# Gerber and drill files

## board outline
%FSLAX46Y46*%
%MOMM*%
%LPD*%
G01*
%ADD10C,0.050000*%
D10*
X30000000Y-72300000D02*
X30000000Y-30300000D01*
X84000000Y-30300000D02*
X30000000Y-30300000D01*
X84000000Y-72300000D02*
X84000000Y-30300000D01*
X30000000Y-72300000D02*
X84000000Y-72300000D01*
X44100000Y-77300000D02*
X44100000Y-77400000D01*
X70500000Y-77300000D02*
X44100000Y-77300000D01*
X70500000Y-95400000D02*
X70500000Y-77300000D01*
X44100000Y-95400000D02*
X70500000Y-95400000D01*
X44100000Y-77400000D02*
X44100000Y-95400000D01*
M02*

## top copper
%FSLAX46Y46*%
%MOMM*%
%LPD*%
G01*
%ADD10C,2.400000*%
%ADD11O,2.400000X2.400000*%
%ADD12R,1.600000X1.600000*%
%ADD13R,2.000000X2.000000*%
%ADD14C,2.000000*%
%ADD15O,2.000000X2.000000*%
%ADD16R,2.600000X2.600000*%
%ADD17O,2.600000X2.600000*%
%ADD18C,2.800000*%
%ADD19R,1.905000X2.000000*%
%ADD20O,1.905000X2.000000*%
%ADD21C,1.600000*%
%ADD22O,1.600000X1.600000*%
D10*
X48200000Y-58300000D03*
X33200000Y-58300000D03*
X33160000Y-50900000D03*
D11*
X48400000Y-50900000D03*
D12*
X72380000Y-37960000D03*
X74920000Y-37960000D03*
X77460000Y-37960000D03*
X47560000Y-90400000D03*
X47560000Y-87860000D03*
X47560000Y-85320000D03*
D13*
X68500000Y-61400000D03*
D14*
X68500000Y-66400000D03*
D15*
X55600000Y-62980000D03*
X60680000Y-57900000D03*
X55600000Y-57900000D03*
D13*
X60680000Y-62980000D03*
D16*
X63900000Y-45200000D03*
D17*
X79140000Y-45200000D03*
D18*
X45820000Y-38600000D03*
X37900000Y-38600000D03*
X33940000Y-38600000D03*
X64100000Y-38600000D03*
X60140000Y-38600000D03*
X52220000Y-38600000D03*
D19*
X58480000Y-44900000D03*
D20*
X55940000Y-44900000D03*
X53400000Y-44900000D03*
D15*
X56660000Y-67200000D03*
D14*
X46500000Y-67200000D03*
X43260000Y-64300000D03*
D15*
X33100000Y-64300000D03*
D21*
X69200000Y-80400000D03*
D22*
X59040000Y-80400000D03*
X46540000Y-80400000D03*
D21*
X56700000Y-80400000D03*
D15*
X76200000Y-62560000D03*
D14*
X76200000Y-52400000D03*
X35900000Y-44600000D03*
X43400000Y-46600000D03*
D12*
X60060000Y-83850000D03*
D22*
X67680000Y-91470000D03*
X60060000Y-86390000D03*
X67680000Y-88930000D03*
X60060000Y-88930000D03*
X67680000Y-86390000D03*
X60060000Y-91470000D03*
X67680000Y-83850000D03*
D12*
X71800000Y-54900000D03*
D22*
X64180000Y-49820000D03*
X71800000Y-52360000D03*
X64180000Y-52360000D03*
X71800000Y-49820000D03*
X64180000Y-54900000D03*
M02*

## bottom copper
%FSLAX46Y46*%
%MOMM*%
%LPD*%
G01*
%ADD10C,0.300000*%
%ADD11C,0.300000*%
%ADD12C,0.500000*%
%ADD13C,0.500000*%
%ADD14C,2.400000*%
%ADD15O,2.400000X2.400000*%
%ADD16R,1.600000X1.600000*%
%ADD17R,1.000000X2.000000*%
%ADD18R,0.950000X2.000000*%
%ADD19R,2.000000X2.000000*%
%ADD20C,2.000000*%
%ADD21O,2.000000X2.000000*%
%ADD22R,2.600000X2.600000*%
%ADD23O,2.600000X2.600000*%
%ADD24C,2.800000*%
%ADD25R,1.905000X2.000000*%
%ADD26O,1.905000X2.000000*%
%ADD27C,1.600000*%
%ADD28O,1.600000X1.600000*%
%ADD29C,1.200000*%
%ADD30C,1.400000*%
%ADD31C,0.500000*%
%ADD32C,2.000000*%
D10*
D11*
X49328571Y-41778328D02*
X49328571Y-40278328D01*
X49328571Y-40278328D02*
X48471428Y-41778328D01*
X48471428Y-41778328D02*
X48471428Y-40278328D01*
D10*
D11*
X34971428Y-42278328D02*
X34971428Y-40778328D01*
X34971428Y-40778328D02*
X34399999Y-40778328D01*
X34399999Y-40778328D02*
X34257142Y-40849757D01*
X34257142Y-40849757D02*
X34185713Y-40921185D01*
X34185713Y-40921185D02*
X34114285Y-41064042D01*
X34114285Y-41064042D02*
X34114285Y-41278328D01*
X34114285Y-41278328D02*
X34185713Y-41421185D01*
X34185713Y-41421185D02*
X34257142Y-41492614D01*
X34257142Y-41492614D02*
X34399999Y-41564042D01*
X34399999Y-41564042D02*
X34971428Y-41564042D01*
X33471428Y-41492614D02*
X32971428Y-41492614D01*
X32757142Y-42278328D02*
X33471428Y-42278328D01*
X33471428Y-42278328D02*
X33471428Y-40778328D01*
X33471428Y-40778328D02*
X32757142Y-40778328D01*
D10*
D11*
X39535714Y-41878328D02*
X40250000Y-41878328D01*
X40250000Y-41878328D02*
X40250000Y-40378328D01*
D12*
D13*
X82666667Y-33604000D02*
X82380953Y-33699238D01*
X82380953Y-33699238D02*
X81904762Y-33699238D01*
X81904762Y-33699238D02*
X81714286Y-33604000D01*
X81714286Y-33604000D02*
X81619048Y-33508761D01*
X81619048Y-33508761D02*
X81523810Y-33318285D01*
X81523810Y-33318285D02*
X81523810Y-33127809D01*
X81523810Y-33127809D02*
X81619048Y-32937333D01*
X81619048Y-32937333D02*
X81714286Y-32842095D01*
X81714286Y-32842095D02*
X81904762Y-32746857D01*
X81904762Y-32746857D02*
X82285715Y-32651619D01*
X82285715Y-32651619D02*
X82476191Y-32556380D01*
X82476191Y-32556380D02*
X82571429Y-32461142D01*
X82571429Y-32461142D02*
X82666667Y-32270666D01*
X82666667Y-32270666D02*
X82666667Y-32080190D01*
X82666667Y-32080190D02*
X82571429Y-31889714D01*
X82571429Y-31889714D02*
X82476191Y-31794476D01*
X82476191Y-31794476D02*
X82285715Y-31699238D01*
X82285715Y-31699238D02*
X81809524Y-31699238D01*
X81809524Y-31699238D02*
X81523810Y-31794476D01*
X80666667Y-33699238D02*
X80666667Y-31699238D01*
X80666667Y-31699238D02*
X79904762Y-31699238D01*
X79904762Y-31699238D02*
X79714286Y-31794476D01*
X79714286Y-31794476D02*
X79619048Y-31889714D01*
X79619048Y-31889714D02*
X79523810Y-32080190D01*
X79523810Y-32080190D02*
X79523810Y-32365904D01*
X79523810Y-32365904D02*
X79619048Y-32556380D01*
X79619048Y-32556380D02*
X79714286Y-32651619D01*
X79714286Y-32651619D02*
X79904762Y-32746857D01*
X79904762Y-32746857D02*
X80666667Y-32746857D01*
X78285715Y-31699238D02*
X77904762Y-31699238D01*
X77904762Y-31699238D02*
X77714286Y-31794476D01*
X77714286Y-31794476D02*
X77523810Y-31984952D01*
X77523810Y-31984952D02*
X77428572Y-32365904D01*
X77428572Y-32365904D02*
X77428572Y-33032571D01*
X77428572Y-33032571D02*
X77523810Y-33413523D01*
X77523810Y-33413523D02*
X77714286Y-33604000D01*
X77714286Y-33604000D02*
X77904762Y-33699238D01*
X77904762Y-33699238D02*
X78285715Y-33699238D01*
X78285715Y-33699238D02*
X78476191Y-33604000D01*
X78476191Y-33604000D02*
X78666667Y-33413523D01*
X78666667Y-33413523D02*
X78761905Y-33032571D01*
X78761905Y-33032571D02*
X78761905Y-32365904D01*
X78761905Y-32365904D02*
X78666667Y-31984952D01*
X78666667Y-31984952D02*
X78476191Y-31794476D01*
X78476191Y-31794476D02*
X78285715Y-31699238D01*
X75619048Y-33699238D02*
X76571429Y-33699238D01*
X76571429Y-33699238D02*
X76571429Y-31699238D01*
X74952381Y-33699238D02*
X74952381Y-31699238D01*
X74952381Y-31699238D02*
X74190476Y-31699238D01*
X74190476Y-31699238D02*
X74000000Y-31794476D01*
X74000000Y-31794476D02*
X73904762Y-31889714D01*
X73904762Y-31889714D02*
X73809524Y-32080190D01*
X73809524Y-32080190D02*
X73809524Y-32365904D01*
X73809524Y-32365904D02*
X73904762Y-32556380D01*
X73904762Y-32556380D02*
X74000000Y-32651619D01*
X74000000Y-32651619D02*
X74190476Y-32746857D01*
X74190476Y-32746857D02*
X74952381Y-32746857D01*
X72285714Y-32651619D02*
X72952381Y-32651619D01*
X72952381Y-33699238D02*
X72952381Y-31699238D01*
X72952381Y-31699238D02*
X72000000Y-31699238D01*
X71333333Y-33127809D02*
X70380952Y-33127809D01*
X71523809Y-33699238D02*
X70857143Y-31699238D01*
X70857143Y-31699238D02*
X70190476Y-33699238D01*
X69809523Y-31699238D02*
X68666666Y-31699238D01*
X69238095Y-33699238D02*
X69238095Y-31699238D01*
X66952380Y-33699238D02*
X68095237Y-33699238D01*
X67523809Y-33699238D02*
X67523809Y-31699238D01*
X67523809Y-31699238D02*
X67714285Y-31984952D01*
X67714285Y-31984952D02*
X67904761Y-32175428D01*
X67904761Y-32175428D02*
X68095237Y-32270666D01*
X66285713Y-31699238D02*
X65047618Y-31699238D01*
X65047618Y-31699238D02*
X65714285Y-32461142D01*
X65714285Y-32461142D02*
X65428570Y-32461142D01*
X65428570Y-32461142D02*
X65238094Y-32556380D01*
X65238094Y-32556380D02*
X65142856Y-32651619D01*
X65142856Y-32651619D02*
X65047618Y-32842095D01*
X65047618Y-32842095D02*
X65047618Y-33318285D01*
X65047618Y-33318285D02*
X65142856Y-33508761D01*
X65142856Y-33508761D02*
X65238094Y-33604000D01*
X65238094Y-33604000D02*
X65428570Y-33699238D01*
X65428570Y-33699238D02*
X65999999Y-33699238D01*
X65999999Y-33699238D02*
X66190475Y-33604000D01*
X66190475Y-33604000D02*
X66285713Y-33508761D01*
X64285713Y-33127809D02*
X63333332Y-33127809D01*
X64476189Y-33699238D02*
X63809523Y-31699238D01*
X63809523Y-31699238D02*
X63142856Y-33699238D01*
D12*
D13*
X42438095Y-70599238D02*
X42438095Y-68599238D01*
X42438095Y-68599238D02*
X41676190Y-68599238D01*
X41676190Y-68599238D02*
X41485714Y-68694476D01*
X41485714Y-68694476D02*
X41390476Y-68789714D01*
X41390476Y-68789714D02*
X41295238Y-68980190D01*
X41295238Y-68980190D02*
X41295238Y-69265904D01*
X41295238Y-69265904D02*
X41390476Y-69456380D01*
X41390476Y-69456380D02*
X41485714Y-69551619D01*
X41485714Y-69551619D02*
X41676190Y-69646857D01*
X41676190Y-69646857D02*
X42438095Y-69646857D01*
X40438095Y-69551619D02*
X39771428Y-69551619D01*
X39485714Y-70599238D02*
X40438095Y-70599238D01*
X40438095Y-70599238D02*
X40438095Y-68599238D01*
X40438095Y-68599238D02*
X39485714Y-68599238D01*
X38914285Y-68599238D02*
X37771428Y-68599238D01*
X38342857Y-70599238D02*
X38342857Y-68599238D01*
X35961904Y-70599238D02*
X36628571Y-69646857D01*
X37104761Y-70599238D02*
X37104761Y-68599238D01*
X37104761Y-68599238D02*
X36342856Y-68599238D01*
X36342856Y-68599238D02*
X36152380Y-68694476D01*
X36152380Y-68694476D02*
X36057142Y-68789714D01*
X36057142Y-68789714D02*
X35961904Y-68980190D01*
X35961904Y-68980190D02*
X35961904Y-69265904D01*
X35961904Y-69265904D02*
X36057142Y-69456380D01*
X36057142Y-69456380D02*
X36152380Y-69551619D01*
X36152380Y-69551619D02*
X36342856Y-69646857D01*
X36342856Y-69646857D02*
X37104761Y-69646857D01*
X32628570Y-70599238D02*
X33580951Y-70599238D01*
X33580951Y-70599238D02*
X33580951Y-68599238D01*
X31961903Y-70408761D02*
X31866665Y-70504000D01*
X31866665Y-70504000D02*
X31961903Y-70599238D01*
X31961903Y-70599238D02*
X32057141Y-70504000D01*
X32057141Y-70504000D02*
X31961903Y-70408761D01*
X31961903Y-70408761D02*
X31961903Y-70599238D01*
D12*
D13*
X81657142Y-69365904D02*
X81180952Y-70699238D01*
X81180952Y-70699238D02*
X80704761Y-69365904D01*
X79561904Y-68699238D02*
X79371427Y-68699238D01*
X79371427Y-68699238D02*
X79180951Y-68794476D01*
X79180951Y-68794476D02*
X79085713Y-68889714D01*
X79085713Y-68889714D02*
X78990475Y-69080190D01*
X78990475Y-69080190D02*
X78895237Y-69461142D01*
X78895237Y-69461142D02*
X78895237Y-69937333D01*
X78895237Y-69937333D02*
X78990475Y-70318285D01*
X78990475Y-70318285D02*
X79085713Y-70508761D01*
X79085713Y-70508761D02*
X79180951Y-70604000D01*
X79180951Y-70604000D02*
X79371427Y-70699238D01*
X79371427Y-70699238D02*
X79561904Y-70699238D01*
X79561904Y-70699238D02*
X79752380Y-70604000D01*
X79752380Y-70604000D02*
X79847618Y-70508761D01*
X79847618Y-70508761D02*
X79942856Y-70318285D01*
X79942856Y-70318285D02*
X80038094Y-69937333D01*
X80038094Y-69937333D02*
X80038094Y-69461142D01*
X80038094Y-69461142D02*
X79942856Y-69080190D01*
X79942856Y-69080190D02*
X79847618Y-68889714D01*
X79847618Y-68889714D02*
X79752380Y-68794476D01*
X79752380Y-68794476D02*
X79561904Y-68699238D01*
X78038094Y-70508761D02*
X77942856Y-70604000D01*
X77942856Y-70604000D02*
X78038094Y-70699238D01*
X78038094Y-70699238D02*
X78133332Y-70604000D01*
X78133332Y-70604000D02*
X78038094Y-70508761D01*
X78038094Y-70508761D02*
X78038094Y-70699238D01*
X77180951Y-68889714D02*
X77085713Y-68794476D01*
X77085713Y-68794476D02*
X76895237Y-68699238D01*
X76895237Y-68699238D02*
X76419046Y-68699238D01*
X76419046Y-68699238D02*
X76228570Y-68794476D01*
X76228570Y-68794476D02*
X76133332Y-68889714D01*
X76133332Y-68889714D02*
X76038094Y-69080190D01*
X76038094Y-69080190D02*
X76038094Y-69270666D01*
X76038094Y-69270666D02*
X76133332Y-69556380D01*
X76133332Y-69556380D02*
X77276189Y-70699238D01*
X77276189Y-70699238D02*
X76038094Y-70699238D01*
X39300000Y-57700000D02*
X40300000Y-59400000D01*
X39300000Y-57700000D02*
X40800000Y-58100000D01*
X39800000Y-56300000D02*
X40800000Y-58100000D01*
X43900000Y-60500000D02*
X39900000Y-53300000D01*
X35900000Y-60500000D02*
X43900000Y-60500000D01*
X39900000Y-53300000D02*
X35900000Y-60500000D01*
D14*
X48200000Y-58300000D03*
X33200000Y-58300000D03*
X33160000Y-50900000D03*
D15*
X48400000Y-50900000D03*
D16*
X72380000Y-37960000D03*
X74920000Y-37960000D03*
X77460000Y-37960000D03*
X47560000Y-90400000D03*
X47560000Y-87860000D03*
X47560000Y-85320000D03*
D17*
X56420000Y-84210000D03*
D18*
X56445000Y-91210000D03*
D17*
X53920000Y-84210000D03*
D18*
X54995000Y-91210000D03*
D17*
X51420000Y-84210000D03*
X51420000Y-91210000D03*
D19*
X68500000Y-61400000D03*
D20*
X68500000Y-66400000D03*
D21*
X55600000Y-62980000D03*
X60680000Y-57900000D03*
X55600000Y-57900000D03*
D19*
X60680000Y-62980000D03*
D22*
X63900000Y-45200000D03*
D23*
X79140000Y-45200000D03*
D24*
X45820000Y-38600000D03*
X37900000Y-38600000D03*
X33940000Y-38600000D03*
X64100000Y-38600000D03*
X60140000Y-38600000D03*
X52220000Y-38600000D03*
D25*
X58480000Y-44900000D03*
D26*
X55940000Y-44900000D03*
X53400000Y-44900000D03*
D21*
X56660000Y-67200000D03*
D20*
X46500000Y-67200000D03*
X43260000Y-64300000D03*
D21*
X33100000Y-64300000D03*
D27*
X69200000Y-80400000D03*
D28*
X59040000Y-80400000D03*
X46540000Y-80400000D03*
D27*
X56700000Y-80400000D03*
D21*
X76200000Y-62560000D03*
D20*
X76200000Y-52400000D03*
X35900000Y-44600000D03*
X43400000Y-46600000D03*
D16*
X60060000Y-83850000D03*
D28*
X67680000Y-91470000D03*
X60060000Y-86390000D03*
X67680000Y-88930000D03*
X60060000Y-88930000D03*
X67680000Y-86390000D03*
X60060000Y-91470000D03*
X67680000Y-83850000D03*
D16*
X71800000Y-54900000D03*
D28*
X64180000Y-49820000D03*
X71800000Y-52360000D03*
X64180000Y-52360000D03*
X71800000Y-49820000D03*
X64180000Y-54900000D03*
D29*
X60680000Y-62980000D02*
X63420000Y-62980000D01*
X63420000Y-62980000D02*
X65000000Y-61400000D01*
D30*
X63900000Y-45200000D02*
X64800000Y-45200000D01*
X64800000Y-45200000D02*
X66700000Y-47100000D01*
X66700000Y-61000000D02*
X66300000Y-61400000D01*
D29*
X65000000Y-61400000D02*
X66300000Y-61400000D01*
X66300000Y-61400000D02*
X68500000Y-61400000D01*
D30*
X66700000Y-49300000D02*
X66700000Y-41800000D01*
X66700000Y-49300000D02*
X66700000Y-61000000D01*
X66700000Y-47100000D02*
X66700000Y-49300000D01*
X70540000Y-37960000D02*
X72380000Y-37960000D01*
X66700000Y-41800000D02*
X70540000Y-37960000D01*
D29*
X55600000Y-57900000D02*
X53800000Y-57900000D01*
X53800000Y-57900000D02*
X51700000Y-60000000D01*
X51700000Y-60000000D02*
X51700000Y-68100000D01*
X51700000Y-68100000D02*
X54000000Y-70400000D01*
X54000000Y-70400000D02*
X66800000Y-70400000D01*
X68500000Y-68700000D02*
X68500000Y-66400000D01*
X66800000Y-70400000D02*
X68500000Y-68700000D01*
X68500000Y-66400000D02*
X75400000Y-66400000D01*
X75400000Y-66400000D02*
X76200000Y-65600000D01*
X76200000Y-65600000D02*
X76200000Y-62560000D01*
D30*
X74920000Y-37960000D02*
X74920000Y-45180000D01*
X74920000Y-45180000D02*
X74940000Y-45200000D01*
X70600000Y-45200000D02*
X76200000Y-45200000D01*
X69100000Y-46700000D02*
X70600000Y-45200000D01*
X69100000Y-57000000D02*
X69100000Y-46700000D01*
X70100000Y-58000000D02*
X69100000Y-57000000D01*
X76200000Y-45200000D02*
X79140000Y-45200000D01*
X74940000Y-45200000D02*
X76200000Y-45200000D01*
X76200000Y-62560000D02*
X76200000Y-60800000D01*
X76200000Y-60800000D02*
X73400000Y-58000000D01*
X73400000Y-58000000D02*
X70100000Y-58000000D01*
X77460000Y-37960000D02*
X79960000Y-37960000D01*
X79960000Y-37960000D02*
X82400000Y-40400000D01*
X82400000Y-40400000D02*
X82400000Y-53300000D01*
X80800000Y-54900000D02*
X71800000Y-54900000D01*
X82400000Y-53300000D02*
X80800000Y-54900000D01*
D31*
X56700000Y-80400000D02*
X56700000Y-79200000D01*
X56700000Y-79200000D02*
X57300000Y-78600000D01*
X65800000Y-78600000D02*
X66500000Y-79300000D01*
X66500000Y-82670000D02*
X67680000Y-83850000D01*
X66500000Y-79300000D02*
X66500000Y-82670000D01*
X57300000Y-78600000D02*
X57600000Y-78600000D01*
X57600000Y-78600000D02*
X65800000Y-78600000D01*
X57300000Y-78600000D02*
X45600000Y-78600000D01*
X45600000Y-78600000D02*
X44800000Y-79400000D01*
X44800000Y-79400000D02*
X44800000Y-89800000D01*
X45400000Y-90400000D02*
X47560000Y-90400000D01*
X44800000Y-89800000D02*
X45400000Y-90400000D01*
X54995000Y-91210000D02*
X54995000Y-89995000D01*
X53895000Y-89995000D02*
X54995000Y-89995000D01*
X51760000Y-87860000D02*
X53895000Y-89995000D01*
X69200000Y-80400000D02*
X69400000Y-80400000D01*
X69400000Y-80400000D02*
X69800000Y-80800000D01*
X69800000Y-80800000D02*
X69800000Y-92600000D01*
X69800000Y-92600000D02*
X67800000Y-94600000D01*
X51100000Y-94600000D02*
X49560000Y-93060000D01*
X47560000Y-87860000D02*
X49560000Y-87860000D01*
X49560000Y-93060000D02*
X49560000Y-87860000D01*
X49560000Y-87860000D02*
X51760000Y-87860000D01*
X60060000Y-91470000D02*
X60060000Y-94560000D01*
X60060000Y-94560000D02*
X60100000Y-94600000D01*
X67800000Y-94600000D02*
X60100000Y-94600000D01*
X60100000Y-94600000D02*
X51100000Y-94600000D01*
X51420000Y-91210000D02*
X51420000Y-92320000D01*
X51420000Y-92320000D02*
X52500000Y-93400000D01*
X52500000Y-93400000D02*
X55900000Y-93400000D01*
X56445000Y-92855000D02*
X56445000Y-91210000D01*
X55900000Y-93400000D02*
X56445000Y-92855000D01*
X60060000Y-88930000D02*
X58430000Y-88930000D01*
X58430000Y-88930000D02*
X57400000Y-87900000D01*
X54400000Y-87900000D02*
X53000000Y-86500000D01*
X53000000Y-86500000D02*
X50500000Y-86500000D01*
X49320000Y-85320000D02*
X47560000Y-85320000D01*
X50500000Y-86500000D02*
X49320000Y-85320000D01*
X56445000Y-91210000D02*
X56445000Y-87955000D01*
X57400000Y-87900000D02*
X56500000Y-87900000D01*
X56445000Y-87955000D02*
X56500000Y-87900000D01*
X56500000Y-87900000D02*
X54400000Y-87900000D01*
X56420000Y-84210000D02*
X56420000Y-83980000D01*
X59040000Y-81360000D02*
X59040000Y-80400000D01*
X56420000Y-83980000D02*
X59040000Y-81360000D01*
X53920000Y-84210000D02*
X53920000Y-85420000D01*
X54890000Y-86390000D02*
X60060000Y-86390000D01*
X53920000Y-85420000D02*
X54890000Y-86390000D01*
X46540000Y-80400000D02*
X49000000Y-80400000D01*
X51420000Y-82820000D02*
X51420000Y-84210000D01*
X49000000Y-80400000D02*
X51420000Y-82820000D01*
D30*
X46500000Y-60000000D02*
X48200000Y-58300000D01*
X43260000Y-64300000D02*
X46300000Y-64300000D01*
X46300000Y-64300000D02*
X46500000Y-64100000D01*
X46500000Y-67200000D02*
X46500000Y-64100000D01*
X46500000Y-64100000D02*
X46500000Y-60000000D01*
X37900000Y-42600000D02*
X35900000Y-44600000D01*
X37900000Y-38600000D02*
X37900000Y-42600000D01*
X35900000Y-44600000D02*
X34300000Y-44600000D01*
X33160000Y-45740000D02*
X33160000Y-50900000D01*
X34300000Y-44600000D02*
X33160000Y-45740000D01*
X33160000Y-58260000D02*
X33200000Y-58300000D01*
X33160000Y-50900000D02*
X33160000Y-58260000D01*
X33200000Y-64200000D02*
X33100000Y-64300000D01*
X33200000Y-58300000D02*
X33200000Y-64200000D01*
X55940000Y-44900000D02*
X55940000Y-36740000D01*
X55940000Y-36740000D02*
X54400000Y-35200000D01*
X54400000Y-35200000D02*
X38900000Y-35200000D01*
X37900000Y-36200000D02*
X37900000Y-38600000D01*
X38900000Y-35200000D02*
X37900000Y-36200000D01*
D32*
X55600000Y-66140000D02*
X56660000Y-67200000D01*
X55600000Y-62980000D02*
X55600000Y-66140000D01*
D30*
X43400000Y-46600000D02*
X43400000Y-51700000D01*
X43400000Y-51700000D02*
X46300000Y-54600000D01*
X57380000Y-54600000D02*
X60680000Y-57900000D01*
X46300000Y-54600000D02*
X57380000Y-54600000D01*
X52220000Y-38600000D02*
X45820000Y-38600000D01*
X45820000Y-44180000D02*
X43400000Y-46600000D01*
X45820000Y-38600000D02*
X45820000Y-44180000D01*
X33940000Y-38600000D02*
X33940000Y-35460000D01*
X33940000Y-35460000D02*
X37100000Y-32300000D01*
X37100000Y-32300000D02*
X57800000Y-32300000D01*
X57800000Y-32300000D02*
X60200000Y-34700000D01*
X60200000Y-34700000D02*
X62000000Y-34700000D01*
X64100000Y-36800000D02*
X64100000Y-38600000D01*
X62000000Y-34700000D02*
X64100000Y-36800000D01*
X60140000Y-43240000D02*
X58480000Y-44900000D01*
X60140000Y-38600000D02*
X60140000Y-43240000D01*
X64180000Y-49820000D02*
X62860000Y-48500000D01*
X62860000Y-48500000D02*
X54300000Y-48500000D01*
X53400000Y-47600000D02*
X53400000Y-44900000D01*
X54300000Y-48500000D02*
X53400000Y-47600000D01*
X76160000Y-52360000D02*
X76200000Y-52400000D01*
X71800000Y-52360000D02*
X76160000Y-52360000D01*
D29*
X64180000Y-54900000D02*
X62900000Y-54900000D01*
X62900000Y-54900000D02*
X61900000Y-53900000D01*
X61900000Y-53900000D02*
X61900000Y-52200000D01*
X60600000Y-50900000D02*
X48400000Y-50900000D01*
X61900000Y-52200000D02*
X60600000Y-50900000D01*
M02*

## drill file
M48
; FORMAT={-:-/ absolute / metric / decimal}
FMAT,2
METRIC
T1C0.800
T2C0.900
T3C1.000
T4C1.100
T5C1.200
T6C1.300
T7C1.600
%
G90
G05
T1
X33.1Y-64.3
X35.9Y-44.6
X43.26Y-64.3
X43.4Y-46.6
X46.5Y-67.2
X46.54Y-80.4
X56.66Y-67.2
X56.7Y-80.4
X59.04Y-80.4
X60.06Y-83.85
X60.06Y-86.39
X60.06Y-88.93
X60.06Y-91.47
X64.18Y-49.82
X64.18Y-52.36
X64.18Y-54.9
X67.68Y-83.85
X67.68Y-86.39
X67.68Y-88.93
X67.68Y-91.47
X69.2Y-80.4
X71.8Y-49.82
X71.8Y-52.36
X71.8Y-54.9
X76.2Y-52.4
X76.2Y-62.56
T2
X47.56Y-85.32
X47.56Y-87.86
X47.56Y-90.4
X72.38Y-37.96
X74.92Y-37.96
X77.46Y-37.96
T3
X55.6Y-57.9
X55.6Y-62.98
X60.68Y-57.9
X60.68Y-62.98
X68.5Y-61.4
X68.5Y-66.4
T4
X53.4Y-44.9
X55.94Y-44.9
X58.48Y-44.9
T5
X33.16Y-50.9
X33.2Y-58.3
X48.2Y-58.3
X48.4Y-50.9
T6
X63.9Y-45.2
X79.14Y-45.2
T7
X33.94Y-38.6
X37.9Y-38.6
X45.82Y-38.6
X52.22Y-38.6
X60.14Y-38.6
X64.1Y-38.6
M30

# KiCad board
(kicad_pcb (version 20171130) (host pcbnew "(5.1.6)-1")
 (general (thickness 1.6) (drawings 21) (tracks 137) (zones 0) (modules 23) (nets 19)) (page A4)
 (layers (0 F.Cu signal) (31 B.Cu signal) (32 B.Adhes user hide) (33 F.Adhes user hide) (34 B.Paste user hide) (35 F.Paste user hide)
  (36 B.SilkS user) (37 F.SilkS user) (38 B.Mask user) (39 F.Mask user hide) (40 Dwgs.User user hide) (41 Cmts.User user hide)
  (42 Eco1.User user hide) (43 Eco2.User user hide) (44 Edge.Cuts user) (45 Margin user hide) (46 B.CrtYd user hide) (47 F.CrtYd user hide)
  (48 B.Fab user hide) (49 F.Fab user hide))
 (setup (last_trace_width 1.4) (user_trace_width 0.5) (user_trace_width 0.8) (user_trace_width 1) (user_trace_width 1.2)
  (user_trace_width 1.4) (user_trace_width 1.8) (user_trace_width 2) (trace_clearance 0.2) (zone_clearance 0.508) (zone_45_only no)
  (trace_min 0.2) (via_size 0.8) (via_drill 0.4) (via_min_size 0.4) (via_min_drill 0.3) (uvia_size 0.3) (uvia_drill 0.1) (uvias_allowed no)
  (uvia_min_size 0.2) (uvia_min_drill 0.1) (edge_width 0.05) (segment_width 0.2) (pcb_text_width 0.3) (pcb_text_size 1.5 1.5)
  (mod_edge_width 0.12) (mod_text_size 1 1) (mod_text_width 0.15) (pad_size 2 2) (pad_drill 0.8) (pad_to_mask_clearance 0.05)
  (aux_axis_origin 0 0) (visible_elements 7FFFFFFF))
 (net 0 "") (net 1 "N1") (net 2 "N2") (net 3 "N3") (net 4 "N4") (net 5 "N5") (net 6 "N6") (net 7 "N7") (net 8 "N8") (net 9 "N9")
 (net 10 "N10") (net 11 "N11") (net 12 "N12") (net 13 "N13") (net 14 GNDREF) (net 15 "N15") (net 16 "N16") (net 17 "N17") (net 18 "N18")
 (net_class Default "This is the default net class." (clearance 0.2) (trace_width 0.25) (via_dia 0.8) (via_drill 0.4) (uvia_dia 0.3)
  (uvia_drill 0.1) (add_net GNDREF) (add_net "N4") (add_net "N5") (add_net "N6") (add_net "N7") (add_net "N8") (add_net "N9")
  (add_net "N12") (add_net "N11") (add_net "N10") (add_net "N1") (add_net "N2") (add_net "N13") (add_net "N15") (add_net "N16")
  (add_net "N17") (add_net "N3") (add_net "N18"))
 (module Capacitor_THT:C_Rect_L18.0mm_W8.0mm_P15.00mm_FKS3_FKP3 (layer F.Cu) (at 48.2 58.3 180)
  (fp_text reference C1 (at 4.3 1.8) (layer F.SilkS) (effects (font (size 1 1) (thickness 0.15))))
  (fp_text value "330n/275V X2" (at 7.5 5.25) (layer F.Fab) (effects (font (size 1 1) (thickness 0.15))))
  (pad 1 thru_hole circle (at 0 0 180) (size 2.4 2.4) (drill 1.2) (layers *.Cu *.Mask) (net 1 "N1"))
  (pad 2 thru_hole circle (at 15 0 180) (size 2.4 2.4) (drill 1.2) (layers *.Cu *.Mask) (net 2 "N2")))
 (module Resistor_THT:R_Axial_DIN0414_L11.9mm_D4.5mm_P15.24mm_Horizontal (layer F.Cu) (at 33.16 50.9)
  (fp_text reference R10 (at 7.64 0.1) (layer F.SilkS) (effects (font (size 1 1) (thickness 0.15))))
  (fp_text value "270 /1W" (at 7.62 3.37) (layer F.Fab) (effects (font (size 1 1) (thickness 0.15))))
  (pad 1 thru_hole circle (at 0 0) (size 2.4 2.4) (drill 1.2) (layers *.Cu *.Mask) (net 2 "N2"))
  (pad 2 thru_hole oval (at 15.24 0) (size 2.4 2.4) (drill 1.2) (layers *.Cu *.Mask) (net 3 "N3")))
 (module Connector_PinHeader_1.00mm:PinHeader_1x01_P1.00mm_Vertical (layer F.Cu) (at 72.38 37.96)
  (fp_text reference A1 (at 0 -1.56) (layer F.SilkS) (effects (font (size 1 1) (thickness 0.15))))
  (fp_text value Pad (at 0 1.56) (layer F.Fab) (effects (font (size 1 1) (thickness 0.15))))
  (pad 1 thru_hole rect (at 0 0) (size 1.6 1.6) (drill 0.9) (layers *.Cu *.Mask) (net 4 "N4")))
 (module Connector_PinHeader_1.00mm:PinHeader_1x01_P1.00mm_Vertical (layer F.Cu) (at 74.92 37.96)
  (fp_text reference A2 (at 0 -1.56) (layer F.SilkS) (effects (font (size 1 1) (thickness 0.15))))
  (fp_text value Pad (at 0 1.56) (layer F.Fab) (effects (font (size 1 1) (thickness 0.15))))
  (pad 1 thru_hole rect (at 0 0) (size 1.6 1.6) (drill 0.9) (layers *.Cu *.Mask) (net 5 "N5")))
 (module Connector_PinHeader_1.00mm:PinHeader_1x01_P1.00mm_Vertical (layer F.Cu) (at 77.46 37.96)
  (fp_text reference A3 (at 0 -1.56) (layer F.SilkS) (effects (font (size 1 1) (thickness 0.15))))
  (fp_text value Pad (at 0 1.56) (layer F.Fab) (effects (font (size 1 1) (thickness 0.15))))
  (pad 1 thru_hole rect (at 0 0) (size 1.6 1.6) (drill 0.9) (layers *.Cu *.Mask) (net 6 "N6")))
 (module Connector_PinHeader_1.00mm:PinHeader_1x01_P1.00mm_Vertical (layer F.Cu) (at 47.56 90.4 90)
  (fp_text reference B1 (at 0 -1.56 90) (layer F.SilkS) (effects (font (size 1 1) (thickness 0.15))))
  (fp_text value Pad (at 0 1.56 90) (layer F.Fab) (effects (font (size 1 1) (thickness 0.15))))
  (pad 1 thru_hole rect (at 0 0 90) (size 1.6 1.6) (drill 0.9) (layers *.Cu *.Mask) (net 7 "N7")))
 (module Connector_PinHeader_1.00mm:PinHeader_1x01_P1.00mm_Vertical (layer F.Cu) (at 47.56 87.86 90)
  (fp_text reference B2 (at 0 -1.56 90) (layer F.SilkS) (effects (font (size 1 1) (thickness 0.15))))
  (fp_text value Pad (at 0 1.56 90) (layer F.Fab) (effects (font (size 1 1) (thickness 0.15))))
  (pad 1 thru_hole rect (at 0 0 90) (size 1.6 1.6) (drill 0.9) (layers *.Cu *.Mask) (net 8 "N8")))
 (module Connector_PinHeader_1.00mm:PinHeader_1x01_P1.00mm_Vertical (layer F.Cu) (at 47.56 85.32 90)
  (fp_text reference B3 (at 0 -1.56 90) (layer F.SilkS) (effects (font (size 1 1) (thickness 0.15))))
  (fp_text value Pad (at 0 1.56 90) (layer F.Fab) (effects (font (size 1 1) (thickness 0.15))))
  (pad 1 thru_hole rect (at 0 0 90) (size 1.6 1.6) (drill 0.9) (layers *.Cu *.Mask) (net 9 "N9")))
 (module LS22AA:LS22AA (layer B.Cu) (at 53.92 87.71)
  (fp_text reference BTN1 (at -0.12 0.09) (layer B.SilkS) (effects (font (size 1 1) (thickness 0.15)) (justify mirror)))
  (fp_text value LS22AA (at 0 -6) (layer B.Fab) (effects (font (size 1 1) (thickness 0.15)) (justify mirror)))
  (pad 6 smd rect (at 2.5 -3.5) (size 1 2) (layers B.Cu B.Paste B.Mask) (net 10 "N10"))
  (pad 5 smd rect (at 2.525 3.5) (size 0.95 2) (layers B.Cu B.Paste B.Mask) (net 9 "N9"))
  (pad 4 smd rect (at 0 -3.5) (size 1 2) (layers B.Cu B.Paste B.Mask) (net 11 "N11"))
  (pad 3 smd rect (at 1.075 3.5) (size 0.95 2) (layers B.Cu B.Paste B.Mask) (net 8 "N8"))
  (pad 2 smd rect (at -2.5 -3.5) (size 1 2) (layers B.Cu B.Paste B.Mask) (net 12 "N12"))
  (pad 1 smd rect (at -2.5 3.5) (size 1 2) (layers B.Cu B.Paste B.Mask) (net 9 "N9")))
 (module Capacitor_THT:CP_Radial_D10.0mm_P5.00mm (layer F.Cu) (at 68.5 61.4 270)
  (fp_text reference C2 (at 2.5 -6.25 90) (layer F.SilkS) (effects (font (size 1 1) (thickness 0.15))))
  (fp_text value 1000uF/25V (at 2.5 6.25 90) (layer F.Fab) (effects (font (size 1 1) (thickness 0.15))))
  (pad 1 thru_hole rect (at 0 0 270) (size 2 2) (drill 1) (layers *.Cu *.Mask) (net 4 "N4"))
  (pad 2 thru_hole circle (at 5 0 270) (size 2 2) (drill 1) (layers *.Cu *.Mask) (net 5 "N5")))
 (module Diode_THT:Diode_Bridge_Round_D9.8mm (layer F.Cu) (at 60.68 62.98 180)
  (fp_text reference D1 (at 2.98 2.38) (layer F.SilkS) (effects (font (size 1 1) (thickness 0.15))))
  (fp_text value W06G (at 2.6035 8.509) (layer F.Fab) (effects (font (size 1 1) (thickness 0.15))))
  (pad 4 thru_hole oval (at 5.08 0 180) (size 2 2) (drill 1) (layers *.Cu *.Mask) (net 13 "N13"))
  (pad 2 thru_hole oval (at 0 5.08 180) (size 2 2) (drill 1) (layers *.Cu *.Mask) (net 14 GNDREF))
  (pad 3 thru_hole oval (at 5.08 5.08 180) (size 2 2) (drill 1) (layers *.Cu *.Mask) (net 5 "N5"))
  (pad 1 thru_hole rect (at 0 0 180) (size 2 2) (drill 1) (layers *.Cu *.Mask) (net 4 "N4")))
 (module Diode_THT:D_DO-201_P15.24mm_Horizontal (layer F.Cu) (at 63.9 45.2)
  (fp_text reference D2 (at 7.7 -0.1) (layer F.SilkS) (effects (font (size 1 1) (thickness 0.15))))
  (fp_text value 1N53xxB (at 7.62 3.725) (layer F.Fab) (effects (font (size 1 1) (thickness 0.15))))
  (pad 1 thru_hole rect (at 0 0) (size 2.6 2.6) (drill 1.3) (layers *.Cu *.Mask) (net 4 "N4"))
  (pad 2 thru_hole oval (at 15.24 0) (size 2.6 2.6) (drill 1.3) (layers *.Cu *.Mask) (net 5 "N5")))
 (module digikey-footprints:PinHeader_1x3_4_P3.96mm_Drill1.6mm (layer F.Cu) (at 33.94 38.6)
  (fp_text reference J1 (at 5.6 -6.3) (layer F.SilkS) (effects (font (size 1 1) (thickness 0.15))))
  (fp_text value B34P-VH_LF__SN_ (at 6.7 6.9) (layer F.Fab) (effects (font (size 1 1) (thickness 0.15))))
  (pad 3 thru_hole circle (at 11.88 0) (size 2.8 2.8) (drill 1.6) (layers *.Cu *.Mask) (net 14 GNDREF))
  (pad 2 thru_hole circle (at 3.96 0) (size 2.8 2.8) (drill 1.6) (layers *.Cu *.Mask) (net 2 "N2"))
  (pad 1 thru_hole circle (at 0 0) (size 2.8 2.8) (drill 1.6) (layers *.Cu *.Mask) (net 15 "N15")))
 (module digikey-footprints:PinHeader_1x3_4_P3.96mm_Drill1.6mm (layer F.Cu) (at 64.1 38.6 180)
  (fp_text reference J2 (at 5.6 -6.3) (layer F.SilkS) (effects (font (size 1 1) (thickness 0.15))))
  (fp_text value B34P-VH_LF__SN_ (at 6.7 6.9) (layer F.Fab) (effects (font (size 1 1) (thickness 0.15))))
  (pad 1 thru_hole circle (at 0 0 180) (size 2.8 2.8) (drill 1.6) (layers *.Cu *.Mask) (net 15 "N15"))
  (pad 2 thru_hole circle (at 3.96 0 180) (size 2.8 2.8) (drill 1.6) (layers *.Cu *.Mask) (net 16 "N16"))
  (pad 3 thru_hole circle (at 11.88 0 180) (size 2.8 2.8) (drill 1.6) (layers *.Cu *.Mask) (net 14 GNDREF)))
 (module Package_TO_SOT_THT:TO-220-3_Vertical (layer F.Cu) (at 58.48 44.9 180)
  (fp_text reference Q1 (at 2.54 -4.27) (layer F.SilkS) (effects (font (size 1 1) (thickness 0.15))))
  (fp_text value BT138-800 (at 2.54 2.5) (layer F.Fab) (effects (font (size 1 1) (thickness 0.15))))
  (pad 1 thru_hole rect (at 0 0 180) (size 1.905 2) (drill 1.1) (layers *.Cu *.Mask) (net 16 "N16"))
  (pad 2 thru_hole oval (at 2.54 0 180) (size 1.905 2) (drill 1.1) (layers *.Cu *.Mask) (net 2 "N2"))
  (pad 3 thru_hole oval (at 5.08 0 180) (size 1.905 2) (drill 1.1) (layers *.Cu *.Mask) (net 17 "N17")))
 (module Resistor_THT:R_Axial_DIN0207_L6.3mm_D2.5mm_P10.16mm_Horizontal (layer F.Cu) (at 46.5 67.2)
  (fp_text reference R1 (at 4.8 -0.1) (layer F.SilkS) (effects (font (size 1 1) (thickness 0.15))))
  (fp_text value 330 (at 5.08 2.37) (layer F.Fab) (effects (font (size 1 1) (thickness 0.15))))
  (pad 2 thru_hole oval (at 10.16 0) (size 2 2) (drill 0.8) (layers *.Cu *.Mask) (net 13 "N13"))
  (pad 1 thru_hole circle (at 0 0) (size 2 2) (drill 0.8) (layers *.Cu *.Mask) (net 1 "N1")))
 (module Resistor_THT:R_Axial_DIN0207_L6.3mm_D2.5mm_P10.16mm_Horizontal (layer F.Cu) (at 43.26 64.3 180)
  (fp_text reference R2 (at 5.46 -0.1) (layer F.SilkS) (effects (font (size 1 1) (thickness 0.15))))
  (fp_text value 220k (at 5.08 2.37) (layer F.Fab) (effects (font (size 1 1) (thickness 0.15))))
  (pad 1 thru_hole circle (at 0 0 180) (size 2 2) (drill 0.8) (layers *.Cu *.Mask) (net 1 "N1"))
  (pad 2 thru_hole oval (at 10.16 0 180) (size 2 2) (drill 0.8) (layers *.Cu *.Mask) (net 2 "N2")))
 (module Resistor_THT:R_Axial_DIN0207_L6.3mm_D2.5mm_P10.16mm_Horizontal (layer F.Cu) (at 69.2 80.4 180)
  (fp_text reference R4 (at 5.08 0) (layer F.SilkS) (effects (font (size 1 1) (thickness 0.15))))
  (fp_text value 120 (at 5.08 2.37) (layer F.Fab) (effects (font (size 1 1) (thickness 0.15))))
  (pad 1 thru_hole circle (at 0 0 180) (size 1.6 1.6) (drill 0.8) (layers *.Cu *.Mask) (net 8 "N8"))
  (pad 2 thru_hole oval (at 10.16 0 180) (size 1.6 1.6) (drill 0.8) (layers *.Cu *.Mask) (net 10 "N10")))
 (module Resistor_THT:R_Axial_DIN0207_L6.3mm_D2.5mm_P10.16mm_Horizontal (layer F.Cu) (at 56.7 80.4 180)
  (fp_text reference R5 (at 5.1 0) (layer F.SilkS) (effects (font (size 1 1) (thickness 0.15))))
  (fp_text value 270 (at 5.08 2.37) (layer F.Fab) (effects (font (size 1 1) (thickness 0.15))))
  (pad 2 thru_hole oval (at 10.16 0 180) (size 1.6 1.6) (drill 0.8) (layers *.Cu *.Mask) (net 12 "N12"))
  (pad 1 thru_hole circle (at 0 0 180) (size 1.6 1.6) (drill 0.8) (layers *.Cu *.Mask) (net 7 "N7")))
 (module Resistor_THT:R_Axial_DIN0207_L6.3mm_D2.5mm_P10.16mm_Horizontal (layer F.Cu) (at 76.2 52.4 270)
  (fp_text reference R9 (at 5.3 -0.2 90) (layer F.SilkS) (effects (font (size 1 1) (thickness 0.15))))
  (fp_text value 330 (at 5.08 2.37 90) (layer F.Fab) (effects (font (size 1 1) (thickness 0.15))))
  (pad 2 thru_hole oval (at 10.16 0 270) (size 2 2) (drill 0.8) (layers *.Cu *.Mask) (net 5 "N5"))
  (pad 1 thru_hole circle (at 0 0 270) (size 2 2) (drill 0.8) (layers *.Cu *.Mask) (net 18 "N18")))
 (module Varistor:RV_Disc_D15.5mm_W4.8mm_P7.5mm (layer F.Cu) (at 35.9 44.6)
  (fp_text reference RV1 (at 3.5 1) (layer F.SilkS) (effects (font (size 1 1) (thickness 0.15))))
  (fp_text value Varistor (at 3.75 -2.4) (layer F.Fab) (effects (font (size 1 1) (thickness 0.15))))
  (pad 1 thru_hole circle (at 0 0) (size 2 2) (drill 0.8) (layers *.Cu *.Mask) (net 2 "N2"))
  (pad 2 thru_hole circle (at 7.5 2) (size 2 2) (drill 0.8) (layers *.Cu *.Mask) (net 14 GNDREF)))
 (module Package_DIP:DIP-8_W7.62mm (layer F.Cu) (at 60.06 83.85)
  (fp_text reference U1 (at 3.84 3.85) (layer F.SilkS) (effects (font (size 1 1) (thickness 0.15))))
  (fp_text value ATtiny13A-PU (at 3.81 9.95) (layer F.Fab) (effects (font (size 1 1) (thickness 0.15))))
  (pad 1 thru_hole rect (at 0 0) (size 1.6 1.6) (drill 0.8) (layers *.Cu *.Mask))
  (pad 5 thru_hole oval (at 7.62 7.62) (size 1.6 1.6) (drill 0.8) (layers *.Cu *.Mask))
  (pad 2 thru_hole oval (at 0 2.54) (size 1.6 1.6) (drill 0.8) (layers *.Cu *.Mask) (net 11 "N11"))
  (pad 6 thru_hole oval (at 7.62 5.08) (size 1.6 1.6) (drill 0.8) (layers *.Cu *.Mask))
  (pad 3 thru_hole oval (at 0 5.08) (size 1.6 1.6) (drill 0.8) (layers *.Cu *.Mask) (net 9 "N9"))
  (pad 7 thru_hole oval (at 7.62 2.54) (size 1.6 1.6) (drill 0.8) (layers *.Cu *.Mask))
  (pad 4 thru_hole oval (at 0 7.62) (size 1.6 1.6) (drill 0.8) (layers *.Cu *.Mask) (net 8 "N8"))
  (pad 8 thru_hole oval (at 7.62 0) (size 1.6 1.6) (drill 0.8) (layers *.Cu *.Mask) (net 7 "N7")))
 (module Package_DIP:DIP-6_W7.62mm (layer F.Cu) (at 71.8 54.9 180)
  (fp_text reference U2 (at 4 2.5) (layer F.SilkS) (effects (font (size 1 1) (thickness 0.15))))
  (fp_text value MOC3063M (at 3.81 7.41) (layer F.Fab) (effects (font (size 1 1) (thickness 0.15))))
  (pad 1 thru_hole rect (at 0 0 180) (size 1.6 1.6) (drill 0.8) (layers *.Cu *.Mask) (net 6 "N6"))
  (pad 4 thru_hole oval (at 7.62 5.08 180) (size 1.6 1.6) (drill 0.8) (layers *.Cu *.Mask) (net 17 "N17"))
  (pad 2 thru_hole oval (at 0 2.54 180) (size 1.6 1.6) (drill 0.8) (layers *.Cu *.Mask) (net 18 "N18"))
  (pad 5 thru_hole oval (at 7.62 2.54 180) (size 1.6 1.6) (drill 0.8) (layers *.Cu *.Mask))
  (pad 3 thru_hole oval (at 0 5.08 180) (size 1.6 1.6) (drill 0.8) (layers *.Cu *.Mask))
  (pad 6 thru_hole oval (at 7.62 0 180) (size 1.6 1.6) (drill 0.8) (layers *.Cu *.Mask) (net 3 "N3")))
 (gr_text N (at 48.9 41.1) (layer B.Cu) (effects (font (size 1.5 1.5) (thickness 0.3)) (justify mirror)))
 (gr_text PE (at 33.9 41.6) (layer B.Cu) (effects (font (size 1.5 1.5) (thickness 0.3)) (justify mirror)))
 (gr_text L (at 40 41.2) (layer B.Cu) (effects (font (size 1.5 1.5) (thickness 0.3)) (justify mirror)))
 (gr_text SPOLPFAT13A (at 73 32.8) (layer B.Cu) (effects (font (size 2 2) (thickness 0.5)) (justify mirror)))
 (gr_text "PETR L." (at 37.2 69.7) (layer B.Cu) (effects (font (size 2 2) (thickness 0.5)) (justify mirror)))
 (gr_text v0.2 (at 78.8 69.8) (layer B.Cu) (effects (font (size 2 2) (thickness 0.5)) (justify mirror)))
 (gr_line (start 39.3 57.7) (end 40.3 59.4) (layer B.Cu) (width 0.5))
 (gr_line (start 39.3 57.7) (end 40.8 58.1) (layer B.Cu) (width 0.5))
 (gr_line (start 39.8 56.3) (end 40.8 58.1) (layer B.Cu) (width 0.5))
 (gr_line (start 43.9 60.5) (end 39.9 53.3) (layer B.Cu) (width 0.5))
 (gr_line (start 35.9 60.5) (end 43.9 60.5) (layer B.Cu) (width 0.5))
 (gr_line (start 39.9 53.3) (end 35.9 60.5) (layer B.Cu) (width 0.5))
 (gr_line (start 30 72.3) (end 30 30.3) (layer Edge.Cuts) (width 0.05))
 (gr_line (start 84 30.3) (end 30 30.3) (layer Edge.Cuts) (width 0.05))
 (gr_line (start 84 72.3) (end 84 30.3) (layer Edge.Cuts) (width 0.05))
 (gr_line (start 30 72.3) (end 84 72.3) (layer Edge.Cuts) (width 0.05))
 (gr_line (start 44.1 77.3) (end 44.1 77.4) (layer Edge.Cuts) (width 0.05))
 (gr_line (start 70.5 77.3) (end 44.1 77.3) (layer Edge.Cuts) (width 0.05))
 (gr_line (start 70.5 95.4) (end 70.5 77.3) (layer Edge.Cuts) (width 0.05))
 (gr_line (start 44.1 95.4) (end 70.5 95.4) (layer Edge.Cuts) (width 0.05))
 (gr_line (start 44.1 77.4) (end 44.1 95.4) (layer Edge.Cuts) (width 0.05))
 (segment (start 60.68 62.98) (end 63.42 62.98) (width 1.2) (layer B.Cu) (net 4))
 (segment (start 63.42 62.98) (end 65 61.4) (width 1.2) (layer B.Cu) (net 4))
 (segment (start 63.9 45.2) (end 64.8 45.2) (width 1.4) (layer B.Cu) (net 4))
 (segment (start 64.8 45.2) (end 66.7 47.1) (width 1.4) (layer B.Cu) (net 4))
 (segment (start 66.7 61) (end 66.3 61.4) (width 1.4) (layer B.Cu) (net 4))
 (segment (start 65 61.4) (end 66.3 61.4) (width 1.2) (layer B.Cu) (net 4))
 (segment (start 66.3 61.4) (end 68.5 61.4) (width 1.2) (layer B.Cu) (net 4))
 (segment (start 66.7 49.3) (end 66.7 41.8) (width 1.4) (layer B.Cu) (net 4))
 (segment (start 66.7 49.3) (end 66.7 61) (width 1.4) (layer B.Cu) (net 4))
 (segment (start 66.7 47.1) (end 66.7 49.3) (width 1.4) (layer B.Cu) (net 4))
 (segment (start 70.54 37.96) (end 72.38 37.96) (width 1.4) (layer B.Cu) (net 4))
 (segment (start 66.7 41.8) (end 70.54 37.96) (width 1.4) (layer B.Cu) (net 4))
 (segment (start 55.6 57.9) (end 53.8 57.9) (width 1.2) (layer B.Cu) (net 5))
 (segment (start 53.8 57.9) (end 51.7 60) (width 1.2) (layer B.Cu) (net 5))
 (segment (start 51.7 60) (end 51.7 68.1) (width 1.2) (layer B.Cu) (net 5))
 (segment (start 51.7 68.1) (end 54 70.4) (width 1.2) (layer B.Cu) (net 5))
 (segment (start 54 70.4) (end 66.8 70.4) (width 1.2) (layer B.Cu) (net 5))
 (segment (start 68.5 68.7) (end 68.5 66.4) (width 1.2) (layer B.Cu) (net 5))
 (segment (start 66.8 70.4) (end 68.5 68.7) (width 1.2) (layer B.Cu) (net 5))
 (segment (start 68.5 66.4) (end 75.4 66.4) (width 1.2) (layer B.Cu) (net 5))
 (segment (start 75.4 66.4) (end 76.2 65.6) (width 1.2) (layer B.Cu) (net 5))
 (segment (start 76.2 65.6) (end 76.2 62.56) (width 1.2) (layer B.Cu) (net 5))
 (segment (start 74.92 37.96) (end 74.92 45.18) (width 1.4) (layer B.Cu) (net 5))
 (segment (start 74.92 45.18) (end 74.94 45.2) (width 1.4) (layer B.Cu) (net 5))
 (segment (start 70.6 45.2) (end 76.2 45.2) (width 1.4) (layer B.Cu) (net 5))
 (segment (start 69.1 46.7) (end 70.6 45.2) (width 1.4) (layer B.Cu) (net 5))
 (segment (start 69.1 57) (end 69.1 46.7) (width 1.4) (layer B.Cu) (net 5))
 (segment (start 70.1 58) (end 69.1 57) (width 1.4) (layer B.Cu) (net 5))
 (segment (start 76.2 45.2) (end 79.14 45.2) (width 1.4) (layer B.Cu) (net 5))
 (segment (start 74.94 45.2) (end 76.2 45.2) (width 1.4) (layer B.Cu) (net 5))
 (segment (start 76.2 62.56) (end 76.2 60.8) (width 1.4) (layer B.Cu) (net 5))
 (segment (start 76.2 60.8) (end 73.4 58) (width 1.4) (layer B.Cu) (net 5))
 (segment (start 73.4 58) (end 70.1 58) (width 1.4) (layer B.Cu) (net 5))
 (segment (start 77.46 37.96) (end 79.96 37.96) (width 1.4) (layer B.Cu) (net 6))
 (segment (start 79.96 37.96) (end 82.4 40.4) (width 1.4) (layer B.Cu) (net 6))
 (segment (start 82.4 40.4) (end 82.4 53.3) (width 1.4) (layer B.Cu) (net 6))
 (segment (start 80.8 54.9) (end 71.8 54.9) (width 1.4) (layer B.Cu) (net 6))
 (segment (start 82.4 53.3) (end 80.8 54.9) (width 1.4) (layer B.Cu) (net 6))
 (segment (start 56.7 80.4) (end 56.7 79.2) (width 0.5) (layer B.Cu) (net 7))
 (segment (start 56.7 79.2) (end 57.3 78.6) (width 0.5) (layer B.Cu) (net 7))
 (segment (start 65.8 78.6) (end 66.5 79.3) (width 0.5) (layer B.Cu) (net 7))
 (segment (start 66.5 82.67) (end 67.68 83.85) (width 0.5) (layer B.Cu) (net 7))
 (segment (start 66.5 79.3) (end 66.5 82.67) (width 0.5) (layer B.Cu) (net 7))
 (segment (start 57.3 78.6) (end 57.6 78.6) (width 0.5) (layer B.Cu) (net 7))
 (segment (start 57.6 78.6) (end 65.8 78.6) (width 0.5) (layer B.Cu) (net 7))
 (segment (start 57.3 78.6) (end 45.6 78.6) (width 0.5) (layer B.Cu) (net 7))
 (segment (start 45.6 78.6) (end 44.8 79.4) (width 0.5) (layer B.Cu) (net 7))
 (segment (start 44.8 79.4) (end 44.8 89.8) (width 0.5) (layer B.Cu) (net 7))
 (segment (start 45.4 90.4) (end 47.56 90.4) (width 0.5) (layer B.Cu) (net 7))
 (segment (start 44.8 89.8) (end 45.4 90.4) (width 0.5) (layer B.Cu) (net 7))
 (segment (start 54.995 91.21) (end 54.995 89.995) (width 0.5) (layer B.Cu) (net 8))
 (segment (start 53.895 89.995) (end 54.995 89.995) (width 0.5) (layer B.Cu) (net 8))
 (segment (start 51.76 87.86) (end 53.895 89.995) (width 0.5) (layer B.Cu) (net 8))
 (segment (start 69.2 80.4) (end 69.4 80.4) (width 0.5) (layer B.Cu) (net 8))
 (segment (start 69.4 80.4) (end 69.8 80.8) (width 0.5) (layer B.Cu) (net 8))
 (segment (start 69.8 80.8) (end 69.8 92.6) (width 0.5) (layer B.Cu) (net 8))
 (segment (start 69.8 92.6) (end 67.8 94.6) (width 0.5) (layer B.Cu) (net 8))
 (segment (start 51.1 94.6) (end 49.56 93.06) (width 0.5) (layer B.Cu) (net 8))
 (segment (start 47.56 87.86) (end 49.56 87.86) (width 0.5) (layer B.Cu) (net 8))
 (segment (start 49.56 93.06) (end 49.56 87.86) (width 0.5) (layer B.Cu) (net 8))
 (segment (start 49.56 87.86) (end 51.76 87.86) (width 0.5) (layer B.Cu) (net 8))
 (segment (start 60.06 91.47) (end 60.06 94.56) (width 0.5) (layer B.Cu) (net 8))
 (segment (start 60.06 94.56) (end 60.1 94.6) (width 0.5) (layer B.Cu) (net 8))
 (segment (start 67.8 94.6) (end 60.1 94.6) (width 0.5) (layer B.Cu) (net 8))
 (segment (start 60.1 94.6) (end 51.1 94.6) (width 0.5) (layer B.Cu) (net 8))
 (segment (start 51.42 91.21) (end 51.42 92.32) (width 0.5) (layer B.Cu) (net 9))
 (segment (start 51.42 92.32) (end 52.5 93.4) (width 0.5) (layer B.Cu) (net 9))
 (segment (start 52.5 93.4) (end 55.9 93.4) (width 0.5) (layer B.Cu) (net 9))
 (segment (start 56.445 92.855) (end 56.445 91.21) (width 0.5) (layer B.Cu) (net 9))
 (segment (start 55.9 93.4) (end 56.445 92.855) (width 0.5) (layer B.Cu) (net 9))
 (segment (start 60.06 88.93) (end 58.43 88.93) (width 0.5) (layer B.Cu) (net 9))
 (segment (start 58.43 88.93) (end 57.4 87.9) (width 0.5) (layer B.Cu) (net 9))
 (segment (start 54.4 87.9) (end 53 86.5) (width 0.5) (layer B.Cu) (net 9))
 (segment (start 53 86.5) (end 50.5 86.5) (width 0.5) (layer B.Cu) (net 9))
 (segment (start 49.32 85.32) (end 47.56 85.32) (width 0.5) (layer B.Cu) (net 9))
 (segment (start 50.5 86.5) (end 49.32 85.32) (width 0.5) (layer B.Cu) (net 9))
 (segment (start 56.445 91.21) (end 56.445 87.955) (width 0.5) (layer B.Cu) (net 9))
 (segment (start 57.4 87.9) (end 56.5 87.9) (width 0.5) (layer B.Cu) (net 9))
 (segment (start 56.445 87.955) (end 56.5 87.9) (width 0.5) (layer B.Cu) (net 9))
 (segment (start 56.5 87.9) (end 54.4 87.9) (width 0.5) (layer B.Cu) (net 9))
 (segment (start 56.42 84.21) (end 56.42 83.98) (width 0.5) (layer B.Cu) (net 10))
 (segment (start 59.04 81.36) (end 59.04 80.4) (width 0.5) (layer B.Cu) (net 10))
 (segment (start 56.42 83.98) (end 59.04 81.36) (width 0.5) (layer B.Cu) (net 10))
 (segment (start 53.92 84.21) (end 53.92 85.42) (width 0.5) (layer B.Cu) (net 11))
 (segment (start 54.89 86.39) (end 60.06 86.39) (width 0.5) (layer B.Cu) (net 11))
 (segment (start 53.92 85.42) (end 54.89 86.39) (width 0.5) (layer B.Cu) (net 11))
 (segment (start 46.54 80.4) (end 49 80.4) (width 0.5) (layer B.Cu) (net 12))
 (segment (start 51.42 82.82) (end 51.42 84.21) (width 0.5) (layer B.Cu) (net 12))
 (segment (start 49 80.4) (end 51.42 82.82) (width 0.5) (layer B.Cu) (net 12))
 (segment (start 46.5 60) (end 48.2 58.3) (width 1.4) (layer B.Cu) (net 1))
 (segment (start 43.26 64.3) (end 46.3 64.3) (width 1.4) (layer B.Cu) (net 1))
 (segment (start 46.3 64.3) (end 46.5 64.1) (width 1.4) (layer B.Cu) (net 1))
 (segment (start 46.5 67.2) (end 46.5 64.1) (width 1.4) (layer B.Cu) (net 1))
 (segment (start 46.5 64.1) (end 46.5 60) (width 1.4) (layer B.Cu) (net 1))
 (segment (start 37.9 42.6) (end 35.9 44.6) (width 1.4) (layer B.Cu) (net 2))
 (segment (start 37.9 38.6) (end 37.9 42.6) (width 1.4) (layer B.Cu) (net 2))
 (segment (start 35.9 44.6) (end 34.3 44.6) (width 1.4) (layer B.Cu) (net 2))
 (segment (start 33.16 45.74) (end 33.16 50.9) (width 1.4) (layer B.Cu) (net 2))
 (segment (start 34.3 44.6) (end 33.16 45.74) (width 1.4) (layer B.Cu) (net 2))
 (segment (start 33.16 58.26) (end 33.2 58.3) (width 1.4) (layer B.Cu) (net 2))
 (segment (start 33.16 50.9) (end 33.16 58.26) (width 1.4) (layer B.Cu) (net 2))
 (segment (start 33.2 64.2) (end 33.1 64.3) (width 1.4) (layer B.Cu) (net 2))
 (segment (start 33.2 58.3) (end 33.2 64.2) (width 1.4) (layer B.Cu) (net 2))
 (segment (start 55.94 44.9) (end 55.94 36.74) (width 1.4) (layer B.Cu) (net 2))
 (segment (start 55.94 36.74) (end 54.4 35.2) (width 1.4) (layer B.Cu) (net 2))
 (segment (start 54.4 35.2) (end 38.9 35.2) (width 1.4) (layer B.Cu) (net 2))
 (segment (start 37.9 36.2) (end 37.9 38.6) (width 1.4) (layer B.Cu) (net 2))
 (segment (start 38.9 35.2) (end 37.9 36.2) (width 1.4) (layer B.Cu) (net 2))
 (segment (start 55.6 66.14) (end 56.66 67.2) (width 2) (layer B.Cu) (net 13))
 (segment (start 55.6 62.98) (end 55.6 66.14) (width 2) (layer B.Cu) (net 13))
 (segment (start 43.4 46.6) (end 43.4 51.7) (width 1.4) (layer B.Cu) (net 14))
 (segment (start 43.4 51.7) (end 46.3 54.6) (width 1.4) (layer B.Cu) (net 14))
 (segment (start 57.38 54.6) (end 60.68 57.9) (width 1.4) (layer B.Cu) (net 14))
 (segment (start 46.3 54.6) (end 57.38 54.6) (width 1.4) (layer B.Cu) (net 14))
 (segment (start 52.22 38.6) (end 45.82 38.6) (width 1.4) (layer B.Cu) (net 14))
 (segment (start 45.82 44.18) (end 43.4 46.6) (width 1.4) (layer B.Cu) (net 14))
 (segment (start 45.82 38.6) (end 45.82 44.18) (width 1.4) (layer B.Cu) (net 14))
 (segment (start 33.94 38.6) (end 33.94 35.46) (width 1.4) (layer B.Cu) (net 15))
 (segment (start 33.94 35.46) (end 37.1 32.3) (width 1.4) (layer B.Cu) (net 15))
 (segment (start 37.1 32.3) (end 57.8 32.3) (width 1.4) (layer B.Cu) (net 15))
 (segment (start 57.8 32.3) (end 60.2 34.7) (width 1.4) (layer B.Cu) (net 15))
 (segment (start 60.2 34.7) (end 62 34.7) (width 1.4) (layer B.Cu) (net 15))
 (segment (start 64.1 36.8) (end 64.1 38.6) (width 1.4) (layer B.Cu) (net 15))
 (segment (start 62 34.7) (end 64.1 36.8) (width 1.4) (layer B.Cu) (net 15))
 (segment (start 60.14 43.24) (end 58.48 44.9) (width 1.4) (layer B.Cu) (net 16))
 (segment (start 60.14 38.6) (end 60.14 43.24) (width 1.4) (layer B.Cu) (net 16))
 (segment (start 64.18 49.82) (end 62.86 48.5) (width 1.4) (layer B.Cu) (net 17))
 (segment (start 62.86 48.5) (end 54.3 48.5) (width 1.4) (layer B.Cu) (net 17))
 (segment (start 53.4 47.6) (end 53.4 44.9) (width 1.4) (layer B.Cu) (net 17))
 (segment (start 54.3 48.5) (end 53.4 47.6) (width 1.4) (layer B.Cu) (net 17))
 (segment (start 76.16 52.36) (end 76.2 52.4) (width 1.4) (layer B.Cu) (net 18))
 (segment (start 71.8 52.36) (end 76.16 52.36) (width 1.4) (layer B.Cu) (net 18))
 (segment (start 64.18 54.9) (end 62.9 54.9) (width 1.2) (layer B.Cu) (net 3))
 (segment (start 62.9 54.9) (end 61.9 53.9) (width 1.2) (layer B.Cu) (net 3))
 (segment (start 61.9 53.9) (end 61.9 52.2) (width 1.2) (layer B.Cu) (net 3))
 (segment (start 60.6 50.9) (end 48.4 50.9) (width 1.2) (layer B.Cu) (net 3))
 (segment (start 61.9 52.2) (end 60.6 50.9) (width 1.2) (layer B.Cu) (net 3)))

